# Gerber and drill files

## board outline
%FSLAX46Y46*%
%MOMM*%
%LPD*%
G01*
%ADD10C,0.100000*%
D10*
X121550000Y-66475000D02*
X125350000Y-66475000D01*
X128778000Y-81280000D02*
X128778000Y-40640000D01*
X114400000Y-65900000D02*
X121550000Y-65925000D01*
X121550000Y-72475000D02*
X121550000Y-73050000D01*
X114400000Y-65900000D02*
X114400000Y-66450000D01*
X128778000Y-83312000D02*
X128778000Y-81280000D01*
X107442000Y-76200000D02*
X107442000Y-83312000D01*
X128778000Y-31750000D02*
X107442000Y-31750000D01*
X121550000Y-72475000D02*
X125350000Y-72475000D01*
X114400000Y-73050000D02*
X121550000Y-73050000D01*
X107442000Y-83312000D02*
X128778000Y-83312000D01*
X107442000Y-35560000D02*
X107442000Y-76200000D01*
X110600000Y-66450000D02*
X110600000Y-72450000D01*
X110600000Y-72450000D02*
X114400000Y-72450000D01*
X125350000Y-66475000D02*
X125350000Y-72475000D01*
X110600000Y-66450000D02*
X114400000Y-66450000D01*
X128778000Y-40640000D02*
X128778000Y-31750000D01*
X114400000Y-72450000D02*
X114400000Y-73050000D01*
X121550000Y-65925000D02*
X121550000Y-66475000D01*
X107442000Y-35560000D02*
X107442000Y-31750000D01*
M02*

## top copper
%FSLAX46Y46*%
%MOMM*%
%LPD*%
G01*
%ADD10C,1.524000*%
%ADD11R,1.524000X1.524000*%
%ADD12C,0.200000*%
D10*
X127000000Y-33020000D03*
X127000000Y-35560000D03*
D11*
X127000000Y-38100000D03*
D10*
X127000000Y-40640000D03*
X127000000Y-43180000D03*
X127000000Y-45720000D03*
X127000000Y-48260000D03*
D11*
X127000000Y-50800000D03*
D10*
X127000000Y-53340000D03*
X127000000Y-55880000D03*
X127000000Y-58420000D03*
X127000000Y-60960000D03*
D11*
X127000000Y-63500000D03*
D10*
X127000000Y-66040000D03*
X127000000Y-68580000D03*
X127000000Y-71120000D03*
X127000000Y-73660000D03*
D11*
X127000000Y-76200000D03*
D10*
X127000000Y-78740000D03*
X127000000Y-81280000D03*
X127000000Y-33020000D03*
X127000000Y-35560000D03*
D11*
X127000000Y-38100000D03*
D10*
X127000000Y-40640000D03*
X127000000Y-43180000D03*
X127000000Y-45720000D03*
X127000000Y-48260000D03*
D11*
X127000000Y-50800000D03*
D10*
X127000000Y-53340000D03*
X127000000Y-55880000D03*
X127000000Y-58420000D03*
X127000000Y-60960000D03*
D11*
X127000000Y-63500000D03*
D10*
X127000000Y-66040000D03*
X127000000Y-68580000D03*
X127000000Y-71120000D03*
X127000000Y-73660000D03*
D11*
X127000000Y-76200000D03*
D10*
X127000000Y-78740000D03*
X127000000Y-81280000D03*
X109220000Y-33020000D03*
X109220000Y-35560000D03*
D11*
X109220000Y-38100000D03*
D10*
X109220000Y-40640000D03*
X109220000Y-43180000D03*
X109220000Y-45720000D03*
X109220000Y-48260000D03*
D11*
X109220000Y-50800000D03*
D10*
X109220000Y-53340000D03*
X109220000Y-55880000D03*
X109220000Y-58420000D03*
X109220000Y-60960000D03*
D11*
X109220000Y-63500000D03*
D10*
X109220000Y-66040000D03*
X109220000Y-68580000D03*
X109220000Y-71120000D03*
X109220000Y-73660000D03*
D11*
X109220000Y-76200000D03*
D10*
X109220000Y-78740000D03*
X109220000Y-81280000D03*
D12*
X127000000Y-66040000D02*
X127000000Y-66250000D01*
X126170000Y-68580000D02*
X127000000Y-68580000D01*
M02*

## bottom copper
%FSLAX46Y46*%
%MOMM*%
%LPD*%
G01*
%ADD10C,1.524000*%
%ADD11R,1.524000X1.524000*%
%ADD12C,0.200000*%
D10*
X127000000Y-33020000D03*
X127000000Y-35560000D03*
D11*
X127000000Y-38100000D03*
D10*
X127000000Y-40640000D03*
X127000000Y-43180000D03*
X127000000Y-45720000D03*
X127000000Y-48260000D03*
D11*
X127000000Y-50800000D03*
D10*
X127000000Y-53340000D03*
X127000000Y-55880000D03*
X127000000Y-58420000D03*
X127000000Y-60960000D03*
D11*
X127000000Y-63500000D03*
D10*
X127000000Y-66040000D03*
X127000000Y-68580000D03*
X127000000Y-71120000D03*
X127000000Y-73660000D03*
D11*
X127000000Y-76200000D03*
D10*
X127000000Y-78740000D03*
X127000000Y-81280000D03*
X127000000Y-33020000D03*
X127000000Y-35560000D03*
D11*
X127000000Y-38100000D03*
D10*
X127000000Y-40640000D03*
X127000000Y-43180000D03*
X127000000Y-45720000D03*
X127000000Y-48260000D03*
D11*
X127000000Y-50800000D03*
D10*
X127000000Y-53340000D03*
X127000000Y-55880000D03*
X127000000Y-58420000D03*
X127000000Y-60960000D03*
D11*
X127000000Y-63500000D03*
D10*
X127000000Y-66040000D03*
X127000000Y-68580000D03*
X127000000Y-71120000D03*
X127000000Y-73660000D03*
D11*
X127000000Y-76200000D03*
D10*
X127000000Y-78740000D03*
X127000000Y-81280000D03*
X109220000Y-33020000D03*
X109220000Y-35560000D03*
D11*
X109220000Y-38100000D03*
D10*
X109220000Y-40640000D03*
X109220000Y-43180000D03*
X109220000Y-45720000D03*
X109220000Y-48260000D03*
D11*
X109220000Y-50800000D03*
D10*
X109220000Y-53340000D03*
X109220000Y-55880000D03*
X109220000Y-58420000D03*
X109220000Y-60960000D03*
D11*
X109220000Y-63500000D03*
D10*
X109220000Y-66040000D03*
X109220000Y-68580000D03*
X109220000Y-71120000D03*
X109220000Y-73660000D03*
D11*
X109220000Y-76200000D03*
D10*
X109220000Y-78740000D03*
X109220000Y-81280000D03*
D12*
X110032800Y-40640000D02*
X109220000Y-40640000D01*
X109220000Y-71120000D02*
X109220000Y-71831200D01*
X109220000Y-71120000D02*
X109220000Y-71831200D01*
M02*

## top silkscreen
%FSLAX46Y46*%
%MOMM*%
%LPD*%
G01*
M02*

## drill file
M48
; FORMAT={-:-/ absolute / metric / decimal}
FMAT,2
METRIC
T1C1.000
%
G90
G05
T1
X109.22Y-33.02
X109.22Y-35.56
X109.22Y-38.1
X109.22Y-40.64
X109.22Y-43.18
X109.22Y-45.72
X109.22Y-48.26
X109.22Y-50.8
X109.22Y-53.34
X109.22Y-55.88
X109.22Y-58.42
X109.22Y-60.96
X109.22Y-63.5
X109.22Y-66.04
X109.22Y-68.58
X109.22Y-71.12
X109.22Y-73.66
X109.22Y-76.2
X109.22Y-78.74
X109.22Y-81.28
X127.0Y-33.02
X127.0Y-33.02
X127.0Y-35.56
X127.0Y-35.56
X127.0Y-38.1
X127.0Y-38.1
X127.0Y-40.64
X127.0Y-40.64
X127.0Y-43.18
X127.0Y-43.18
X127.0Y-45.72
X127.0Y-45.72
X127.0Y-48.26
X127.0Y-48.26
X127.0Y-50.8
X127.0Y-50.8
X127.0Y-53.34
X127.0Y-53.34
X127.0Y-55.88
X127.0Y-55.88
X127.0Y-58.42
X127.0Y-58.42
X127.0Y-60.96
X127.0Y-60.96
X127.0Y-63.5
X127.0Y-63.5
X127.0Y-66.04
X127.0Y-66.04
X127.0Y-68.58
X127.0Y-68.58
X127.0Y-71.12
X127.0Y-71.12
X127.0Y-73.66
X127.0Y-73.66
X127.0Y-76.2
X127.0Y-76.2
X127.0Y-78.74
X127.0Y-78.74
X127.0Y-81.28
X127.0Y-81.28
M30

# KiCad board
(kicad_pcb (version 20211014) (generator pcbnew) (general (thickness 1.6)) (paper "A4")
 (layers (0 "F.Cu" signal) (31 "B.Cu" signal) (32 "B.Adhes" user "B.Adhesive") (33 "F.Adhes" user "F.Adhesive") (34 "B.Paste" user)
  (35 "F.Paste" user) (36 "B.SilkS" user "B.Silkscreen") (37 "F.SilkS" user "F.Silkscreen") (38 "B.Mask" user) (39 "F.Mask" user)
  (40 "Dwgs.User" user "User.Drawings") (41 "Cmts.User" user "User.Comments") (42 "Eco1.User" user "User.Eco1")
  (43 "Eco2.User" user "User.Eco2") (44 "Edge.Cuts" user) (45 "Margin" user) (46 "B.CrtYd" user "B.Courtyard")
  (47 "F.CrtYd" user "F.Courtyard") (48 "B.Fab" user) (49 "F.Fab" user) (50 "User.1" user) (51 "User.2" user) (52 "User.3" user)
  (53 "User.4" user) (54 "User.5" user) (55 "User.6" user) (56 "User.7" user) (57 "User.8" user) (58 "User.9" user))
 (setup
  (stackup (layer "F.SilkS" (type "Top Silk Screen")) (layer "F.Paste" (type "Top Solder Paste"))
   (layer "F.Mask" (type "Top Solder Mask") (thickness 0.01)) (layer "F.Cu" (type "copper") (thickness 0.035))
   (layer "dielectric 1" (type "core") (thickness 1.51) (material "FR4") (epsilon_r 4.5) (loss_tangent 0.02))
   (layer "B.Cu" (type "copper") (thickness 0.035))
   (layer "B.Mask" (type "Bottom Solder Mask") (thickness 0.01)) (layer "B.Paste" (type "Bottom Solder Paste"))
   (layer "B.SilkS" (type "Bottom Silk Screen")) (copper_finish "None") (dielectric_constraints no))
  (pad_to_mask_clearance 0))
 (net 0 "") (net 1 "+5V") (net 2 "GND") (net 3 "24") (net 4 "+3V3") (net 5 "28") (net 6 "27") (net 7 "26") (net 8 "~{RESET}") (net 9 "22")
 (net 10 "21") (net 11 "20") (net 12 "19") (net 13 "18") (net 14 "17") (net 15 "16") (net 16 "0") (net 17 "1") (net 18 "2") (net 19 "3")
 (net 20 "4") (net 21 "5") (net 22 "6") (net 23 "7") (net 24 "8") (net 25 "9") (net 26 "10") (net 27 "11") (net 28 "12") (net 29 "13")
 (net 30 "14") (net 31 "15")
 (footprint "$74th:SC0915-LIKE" (layer "F.Cu") (at 127 48.26)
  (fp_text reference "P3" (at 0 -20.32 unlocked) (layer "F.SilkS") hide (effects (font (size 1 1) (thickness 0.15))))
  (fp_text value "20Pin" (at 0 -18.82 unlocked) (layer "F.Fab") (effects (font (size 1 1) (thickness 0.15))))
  (pad "1" thru_hole circle (at 0 -15.24) (size 1.524 1.524) (drill 1) (layers *.Cu *.Mask) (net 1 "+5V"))
  (pad "2" thru_hole circle (at 0 -12.7 180) (size 1.524 1.524) (drill 1) (layers *.Cu *.Mask) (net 1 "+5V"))
  (pad "3" thru_hole rect (at 0 -10.16) (size 1.524 1.524) (drill 1) (layers *.Cu *.Mask) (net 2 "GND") (zone_connect 2))
  (pad "4" thru_hole circle (at 0 -7.62) (size 1.524 1.524) (drill 1) (layers *.Cu *.Mask) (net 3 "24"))
  (pad "5" thru_hole circle (at 0 -5.08) (size 1.524 1.524) (drill 1) (layers *.Cu *.Mask) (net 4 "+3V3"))
  (pad "6" thru_hole circle (at 0 -2.54) (size 1.524 1.524) (drill 1) (layers *.Cu *.Mask) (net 4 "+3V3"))
  (pad "7" thru_hole circle (at 0 0) (size 1.524 1.524) (drill 1) (layers *.Cu *.Mask) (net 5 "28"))
  (pad "8" thru_hole rect (at 0 2.54) (size 1.524 1.524) (drill 1) (layers *.Cu *.Mask) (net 2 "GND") (zone_connect 2))
  (pad "9" thru_hole circle (at 0 5.08) (size 1.524 1.524) (drill 1) (layers *.Cu *.Mask) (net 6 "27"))
  (pad "10" thru_hole circle (at 0 7.62) (size 1.524 1.524) (drill 1) (layers *.Cu *.Mask) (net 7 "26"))
  (pad "11" thru_hole circle (at 0 10.16) (size 1.524 1.524) (drill 1) (layers *.Cu *.Mask) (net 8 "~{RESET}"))
  (pad "12" thru_hole circle (at 0 12.7) (size 1.524 1.524) (drill 1) (layers *.Cu *.Mask) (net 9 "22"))
  (pad "13" thru_hole rect (at 0 15.24) (size 1.524 1.524) (drill 1) (layers *.Cu *.Mask) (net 2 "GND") (zone_connect 2))
  (pad "14" thru_hole circle (at 0 17.78) (size 1.524 1.524) (drill 1) (layers *.Cu *.Mask) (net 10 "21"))
  (pad "15" thru_hole circle (at 0 20.32) (size 1.524 1.524) (drill 1) (layers *.Cu *.Mask) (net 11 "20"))
  (pad "16" thru_hole circle (at 0 22.86) (size 1.524 1.524) (drill 1) (layers *.Cu *.Mask) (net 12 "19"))
  (pad "17" thru_hole circle (at 0 25.4) (size 1.524 1.524) (drill 1) (layers *.Cu *.Mask) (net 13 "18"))
  (pad "18" thru_hole rect (at 0 27.94) (size 1.524 1.524) (drill 1) (layers *.Cu *.Mask) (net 2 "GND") (zone_connect 2))
  (pad "19" thru_hole circle (at 0 30.48) (size 1.524 1.524) (drill 1) (layers *.Cu *.Mask) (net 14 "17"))
  (pad "20" thru_hole circle (at 0 33.02) (size 1.524 1.524) (drill 1) (layers *.Cu *.Mask) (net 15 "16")))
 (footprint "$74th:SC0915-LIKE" (layer "F.Cu") (at 127 48.26)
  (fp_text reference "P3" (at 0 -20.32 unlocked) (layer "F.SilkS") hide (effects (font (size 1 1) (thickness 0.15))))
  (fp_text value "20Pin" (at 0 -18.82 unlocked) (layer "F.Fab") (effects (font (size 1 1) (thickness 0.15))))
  (pad "1" thru_hole circle (at 0 -15.24) (size 1.524 1.524) (drill 1) (layers *.Cu *.Mask) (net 1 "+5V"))
  (pad "2" thru_hole circle (at 0 -12.7 180) (size 1.524 1.524) (drill 1) (layers *.Cu *.Mask) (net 1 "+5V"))
  (pad "3" thru_hole rect (at 0 -10.16) (size 1.524 1.524) (drill 1) (layers *.Cu *.Mask) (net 2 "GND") (zone_connect 2))
  (pad "4" thru_hole circle (at 0 -7.62) (size 1.524 1.524) (drill 1) (layers *.Cu *.Mask) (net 3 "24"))
  (pad "5" thru_hole circle (at 0 -5.08) (size 1.524 1.524) (drill 1) (layers *.Cu *.Mask) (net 4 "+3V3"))
  (pad "6" thru_hole circle (at 0 -2.54) (size 1.524 1.524) (drill 1) (layers *.Cu *.Mask) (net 4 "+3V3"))
  (pad "7" thru_hole circle (at 0 0) (size 1.524 1.524) (drill 1) (layers *.Cu *.Mask) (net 5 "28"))
  (pad "8" thru_hole rect (at 0 2.54) (size 1.524 1.524) (drill 1) (layers *.Cu *.Mask) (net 2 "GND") (zone_connect 2))
  (pad "9" thru_hole circle (at 0 5.08) (size 1.524 1.524) (drill 1) (layers *.Cu *.Mask) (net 6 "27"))
  (pad "10" thru_hole circle (at 0 7.62) (size 1.524 1.524) (drill 1) (layers *.Cu *.Mask) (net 7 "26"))
  (pad "11" thru_hole circle (at 0 10.16) (size 1.524 1.524) (drill 1) (layers *.Cu *.Mask) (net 8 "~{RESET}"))
  (pad "12" thru_hole circle (at 0 12.7) (size 1.524 1.524) (drill 1) (layers *.Cu *.Mask) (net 9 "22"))
  (pad "13" thru_hole rect (at 0 15.24) (size 1.524 1.524) (drill 1) (layers *.Cu *.Mask) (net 2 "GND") (zone_connect 2))
  (pad "14" thru_hole circle (at 0 17.78) (size 1.524 1.524) (drill 1) (layers *.Cu *.Mask) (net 10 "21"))
  (pad "15" thru_hole circle (at 0 20.32) (size 1.524 1.524) (drill 1) (layers *.Cu *.Mask) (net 11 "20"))
  (pad "16" thru_hole circle (at 0 22.86) (size 1.524 1.524) (drill 1) (layers *.Cu *.Mask) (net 12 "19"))
  (pad "17" thru_hole circle (at 0 25.4) (size 1.524 1.524) (drill 1) (layers *.Cu *.Mask) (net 13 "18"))
  (pad "18" thru_hole rect (at 0 27.94) (size 1.524 1.524) (drill 1) (layers *.Cu *.Mask) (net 2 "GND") (zone_connect 2))
  (pad "19" thru_hole circle (at 0 30.48) (size 1.524 1.524) (drill 1) (layers *.Cu *.Mask) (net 14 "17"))
  (pad "20" thru_hole circle (at 0 33.02) (size 1.524 1.524) (drill 1) (layers *.Cu *.Mask) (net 15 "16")))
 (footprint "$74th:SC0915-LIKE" (layer "F.Cu") (at 109.22 48.26)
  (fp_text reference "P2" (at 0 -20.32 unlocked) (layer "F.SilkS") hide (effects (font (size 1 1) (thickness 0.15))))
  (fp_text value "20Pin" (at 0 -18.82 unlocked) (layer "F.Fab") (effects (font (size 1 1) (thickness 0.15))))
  (pad "1" thru_hole circle (at 0 -15.24) (size 1.524 1.524) (drill 1) (layers *.Cu *.Mask) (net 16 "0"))
  (pad "2" thru_hole circle (at 0 -12.7 180) (size 1.524 1.524) (drill 1) (layers *.Cu *.Mask) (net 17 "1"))
  (pad "3" thru_hole rect (at 0 -10.16) (size 1.524 1.524) (drill 1) (layers *.Cu *.Mask) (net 2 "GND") (zone_connect 2))
  (pad "4" thru_hole circle (at 0 -7.62) (size 1.524 1.524) (drill 1) (layers *.Cu *.Mask) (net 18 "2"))
  (pad "5" thru_hole circle (at 0 -5.08) (size 1.524 1.524) (drill 1) (layers *.Cu *.Mask) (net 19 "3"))
  (pad "6" thru_hole circle (at 0 -2.54) (size 1.524 1.524) (drill 1) (layers *.Cu *.Mask) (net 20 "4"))
  (pad "7" thru_hole circle (at 0 0) (size 1.524 1.524) (drill 1) (layers *.Cu *.Mask) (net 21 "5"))
  (pad "8" thru_hole rect (at 0 2.54) (size 1.524 1.524) (drill 1) (layers *.Cu *.Mask) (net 2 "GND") (zone_connect 2))
  (pad "9" thru_hole circle (at 0 5.08) (size 1.524 1.524) (drill 1) (layers *.Cu *.Mask) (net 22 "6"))
  (pad "10" thru_hole circle (at 0 7.62) (size 1.524 1.524) (drill 1) (layers *.Cu *.Mask) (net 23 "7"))
  (pad "11" thru_hole circle (at 0 10.16) (size 1.524 1.524) (drill 1) (layers *.Cu *.Mask) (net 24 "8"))
  (pad "12" thru_hole circle (at 0 12.7) (size 1.524 1.524) (drill 1) (layers *.Cu *.Mask) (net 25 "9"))
  (pad "13" thru_hole rect (at 0 15.24) (size 1.524 1.524) (drill 1) (layers *.Cu *.Mask) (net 2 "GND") (zone_connect 2))
  (pad "14" thru_hole circle (at 0 17.78) (size 1.524 1.524) (drill 1) (layers *.Cu *.Mask) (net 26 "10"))
  (pad "15" thru_hole circle (at 0 20.32) (size 1.524 1.524) (drill 1) (layers *.Cu *.Mask) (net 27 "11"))
  (pad "16" thru_hole circle (at 0 22.86) (size 1.524 1.524) (drill 1) (layers *.Cu *.Mask) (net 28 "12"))
  (pad "17" thru_hole circle (at 0 25.4) (size 1.524 1.524) (drill 1) (layers *.Cu *.Mask) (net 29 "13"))
  (pad "18" thru_hole rect (at 0 27.94) (size 1.524 1.524) (drill 1) (layers *.Cu *.Mask) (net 2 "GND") (zone_connect 2))
  (pad "19" thru_hole circle (at 0 30.48) (size 1.524 1.524) (drill 1) (layers *.Cu *.Mask) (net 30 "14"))
  (pad "20" thru_hole circle (at 0 33.02) (size 1.524 1.524) (drill 1) (layers *.Cu *.Mask) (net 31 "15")))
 (gr_line (start 121.55 66.475) (end 125.35 66.475) (layer "Edge.Cuts") (width 0.1))
 (gr_line (start 128.778 81.28) (end 128.778 40.64) (layer "Edge.Cuts") (width 0.1))
 (gr_line (start 114.4 65.9) (end 121.55 65.925) (layer "Edge.Cuts") (width 0.1))
 (gr_line (start 121.55 72.475) (end 121.55 73.05) (layer "Edge.Cuts") (width 0.1))
 (gr_line (start 114.4 65.9) (end 114.4 66.45) (layer "Edge.Cuts") (width 0.1))
 (gr_line (start 128.778 83.312) (end 128.778 81.28) (layer "Edge.Cuts") (width 0.1))
 (gr_line (start 107.442 76.2) (end 107.442 83.312) (layer "Edge.Cuts") (width 0.1))
 (gr_line (start 128.778 31.75) (end 107.442 31.75) (layer "Edge.Cuts") (width 0.1))
 (gr_line (start 121.55 72.475) (end 125.35 72.475) (layer "Edge.Cuts") (width 0.1))
 (gr_line (start 114.4 73.05) (end 121.55 73.05) (layer "Edge.Cuts") (width 0.1))
 (gr_line (start 107.442 83.312) (end 128.778 83.312) (layer "Edge.Cuts") (width 0.1))
 (gr_line (start 107.442 35.56) (end 107.442 76.2) (layer "Edge.Cuts") (width 0.1))
 (gr_line (start 110.6 66.45) (end 110.6 72.45) (layer "Edge.Cuts") (width 0.1))
 (gr_line (start 110.6 72.45) (end 114.4 72.45) (layer "Edge.Cuts") (width 0.1))
 (gr_line (start 125.35 66.475) (end 125.35 72.475) (layer "Edge.Cuts") (width 0.1))
 (gr_line (start 110.6 66.45) (end 114.4 66.45) (layer "Edge.Cuts") (width 0.1))
 (gr_line (start 128.778 40.64) (end 128.778 31.75) (layer "Edge.Cuts") (width 0.1))
 (gr_line (start 114.4 72.45) (end 114.4 73.05) (layer "Edge.Cuts") (width 0.1))
 (gr_line (start 121.55 65.925) (end 121.55 66.475) (layer "Edge.Cuts") (width 0.1))
 (gr_line (start 107.442 35.56) (end 107.442 31.75) (layer "Edge.Cuts") (width 0.1))
 (segment (start 110.0328 40.64) (end 109.22 40.64) (width 0.2) (layer "B.Cu") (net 18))
 (segment (start 109.22 71.12) (end 109.22 71.8312) (width 0.2) (layer "B.Cu") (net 28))
 (segment (start 109.22 71.12) (end 109.22 71.8312) (width 0.2) (layer "B.Cu") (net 28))
 (segment (start 127 66.04) (end 127 66.25) (width 0.2) (layer "F.Cu") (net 10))
 (segment (start 126.17 68.58) (end 127 68.58) (width 0.2) (layer "F.Cu") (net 11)))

